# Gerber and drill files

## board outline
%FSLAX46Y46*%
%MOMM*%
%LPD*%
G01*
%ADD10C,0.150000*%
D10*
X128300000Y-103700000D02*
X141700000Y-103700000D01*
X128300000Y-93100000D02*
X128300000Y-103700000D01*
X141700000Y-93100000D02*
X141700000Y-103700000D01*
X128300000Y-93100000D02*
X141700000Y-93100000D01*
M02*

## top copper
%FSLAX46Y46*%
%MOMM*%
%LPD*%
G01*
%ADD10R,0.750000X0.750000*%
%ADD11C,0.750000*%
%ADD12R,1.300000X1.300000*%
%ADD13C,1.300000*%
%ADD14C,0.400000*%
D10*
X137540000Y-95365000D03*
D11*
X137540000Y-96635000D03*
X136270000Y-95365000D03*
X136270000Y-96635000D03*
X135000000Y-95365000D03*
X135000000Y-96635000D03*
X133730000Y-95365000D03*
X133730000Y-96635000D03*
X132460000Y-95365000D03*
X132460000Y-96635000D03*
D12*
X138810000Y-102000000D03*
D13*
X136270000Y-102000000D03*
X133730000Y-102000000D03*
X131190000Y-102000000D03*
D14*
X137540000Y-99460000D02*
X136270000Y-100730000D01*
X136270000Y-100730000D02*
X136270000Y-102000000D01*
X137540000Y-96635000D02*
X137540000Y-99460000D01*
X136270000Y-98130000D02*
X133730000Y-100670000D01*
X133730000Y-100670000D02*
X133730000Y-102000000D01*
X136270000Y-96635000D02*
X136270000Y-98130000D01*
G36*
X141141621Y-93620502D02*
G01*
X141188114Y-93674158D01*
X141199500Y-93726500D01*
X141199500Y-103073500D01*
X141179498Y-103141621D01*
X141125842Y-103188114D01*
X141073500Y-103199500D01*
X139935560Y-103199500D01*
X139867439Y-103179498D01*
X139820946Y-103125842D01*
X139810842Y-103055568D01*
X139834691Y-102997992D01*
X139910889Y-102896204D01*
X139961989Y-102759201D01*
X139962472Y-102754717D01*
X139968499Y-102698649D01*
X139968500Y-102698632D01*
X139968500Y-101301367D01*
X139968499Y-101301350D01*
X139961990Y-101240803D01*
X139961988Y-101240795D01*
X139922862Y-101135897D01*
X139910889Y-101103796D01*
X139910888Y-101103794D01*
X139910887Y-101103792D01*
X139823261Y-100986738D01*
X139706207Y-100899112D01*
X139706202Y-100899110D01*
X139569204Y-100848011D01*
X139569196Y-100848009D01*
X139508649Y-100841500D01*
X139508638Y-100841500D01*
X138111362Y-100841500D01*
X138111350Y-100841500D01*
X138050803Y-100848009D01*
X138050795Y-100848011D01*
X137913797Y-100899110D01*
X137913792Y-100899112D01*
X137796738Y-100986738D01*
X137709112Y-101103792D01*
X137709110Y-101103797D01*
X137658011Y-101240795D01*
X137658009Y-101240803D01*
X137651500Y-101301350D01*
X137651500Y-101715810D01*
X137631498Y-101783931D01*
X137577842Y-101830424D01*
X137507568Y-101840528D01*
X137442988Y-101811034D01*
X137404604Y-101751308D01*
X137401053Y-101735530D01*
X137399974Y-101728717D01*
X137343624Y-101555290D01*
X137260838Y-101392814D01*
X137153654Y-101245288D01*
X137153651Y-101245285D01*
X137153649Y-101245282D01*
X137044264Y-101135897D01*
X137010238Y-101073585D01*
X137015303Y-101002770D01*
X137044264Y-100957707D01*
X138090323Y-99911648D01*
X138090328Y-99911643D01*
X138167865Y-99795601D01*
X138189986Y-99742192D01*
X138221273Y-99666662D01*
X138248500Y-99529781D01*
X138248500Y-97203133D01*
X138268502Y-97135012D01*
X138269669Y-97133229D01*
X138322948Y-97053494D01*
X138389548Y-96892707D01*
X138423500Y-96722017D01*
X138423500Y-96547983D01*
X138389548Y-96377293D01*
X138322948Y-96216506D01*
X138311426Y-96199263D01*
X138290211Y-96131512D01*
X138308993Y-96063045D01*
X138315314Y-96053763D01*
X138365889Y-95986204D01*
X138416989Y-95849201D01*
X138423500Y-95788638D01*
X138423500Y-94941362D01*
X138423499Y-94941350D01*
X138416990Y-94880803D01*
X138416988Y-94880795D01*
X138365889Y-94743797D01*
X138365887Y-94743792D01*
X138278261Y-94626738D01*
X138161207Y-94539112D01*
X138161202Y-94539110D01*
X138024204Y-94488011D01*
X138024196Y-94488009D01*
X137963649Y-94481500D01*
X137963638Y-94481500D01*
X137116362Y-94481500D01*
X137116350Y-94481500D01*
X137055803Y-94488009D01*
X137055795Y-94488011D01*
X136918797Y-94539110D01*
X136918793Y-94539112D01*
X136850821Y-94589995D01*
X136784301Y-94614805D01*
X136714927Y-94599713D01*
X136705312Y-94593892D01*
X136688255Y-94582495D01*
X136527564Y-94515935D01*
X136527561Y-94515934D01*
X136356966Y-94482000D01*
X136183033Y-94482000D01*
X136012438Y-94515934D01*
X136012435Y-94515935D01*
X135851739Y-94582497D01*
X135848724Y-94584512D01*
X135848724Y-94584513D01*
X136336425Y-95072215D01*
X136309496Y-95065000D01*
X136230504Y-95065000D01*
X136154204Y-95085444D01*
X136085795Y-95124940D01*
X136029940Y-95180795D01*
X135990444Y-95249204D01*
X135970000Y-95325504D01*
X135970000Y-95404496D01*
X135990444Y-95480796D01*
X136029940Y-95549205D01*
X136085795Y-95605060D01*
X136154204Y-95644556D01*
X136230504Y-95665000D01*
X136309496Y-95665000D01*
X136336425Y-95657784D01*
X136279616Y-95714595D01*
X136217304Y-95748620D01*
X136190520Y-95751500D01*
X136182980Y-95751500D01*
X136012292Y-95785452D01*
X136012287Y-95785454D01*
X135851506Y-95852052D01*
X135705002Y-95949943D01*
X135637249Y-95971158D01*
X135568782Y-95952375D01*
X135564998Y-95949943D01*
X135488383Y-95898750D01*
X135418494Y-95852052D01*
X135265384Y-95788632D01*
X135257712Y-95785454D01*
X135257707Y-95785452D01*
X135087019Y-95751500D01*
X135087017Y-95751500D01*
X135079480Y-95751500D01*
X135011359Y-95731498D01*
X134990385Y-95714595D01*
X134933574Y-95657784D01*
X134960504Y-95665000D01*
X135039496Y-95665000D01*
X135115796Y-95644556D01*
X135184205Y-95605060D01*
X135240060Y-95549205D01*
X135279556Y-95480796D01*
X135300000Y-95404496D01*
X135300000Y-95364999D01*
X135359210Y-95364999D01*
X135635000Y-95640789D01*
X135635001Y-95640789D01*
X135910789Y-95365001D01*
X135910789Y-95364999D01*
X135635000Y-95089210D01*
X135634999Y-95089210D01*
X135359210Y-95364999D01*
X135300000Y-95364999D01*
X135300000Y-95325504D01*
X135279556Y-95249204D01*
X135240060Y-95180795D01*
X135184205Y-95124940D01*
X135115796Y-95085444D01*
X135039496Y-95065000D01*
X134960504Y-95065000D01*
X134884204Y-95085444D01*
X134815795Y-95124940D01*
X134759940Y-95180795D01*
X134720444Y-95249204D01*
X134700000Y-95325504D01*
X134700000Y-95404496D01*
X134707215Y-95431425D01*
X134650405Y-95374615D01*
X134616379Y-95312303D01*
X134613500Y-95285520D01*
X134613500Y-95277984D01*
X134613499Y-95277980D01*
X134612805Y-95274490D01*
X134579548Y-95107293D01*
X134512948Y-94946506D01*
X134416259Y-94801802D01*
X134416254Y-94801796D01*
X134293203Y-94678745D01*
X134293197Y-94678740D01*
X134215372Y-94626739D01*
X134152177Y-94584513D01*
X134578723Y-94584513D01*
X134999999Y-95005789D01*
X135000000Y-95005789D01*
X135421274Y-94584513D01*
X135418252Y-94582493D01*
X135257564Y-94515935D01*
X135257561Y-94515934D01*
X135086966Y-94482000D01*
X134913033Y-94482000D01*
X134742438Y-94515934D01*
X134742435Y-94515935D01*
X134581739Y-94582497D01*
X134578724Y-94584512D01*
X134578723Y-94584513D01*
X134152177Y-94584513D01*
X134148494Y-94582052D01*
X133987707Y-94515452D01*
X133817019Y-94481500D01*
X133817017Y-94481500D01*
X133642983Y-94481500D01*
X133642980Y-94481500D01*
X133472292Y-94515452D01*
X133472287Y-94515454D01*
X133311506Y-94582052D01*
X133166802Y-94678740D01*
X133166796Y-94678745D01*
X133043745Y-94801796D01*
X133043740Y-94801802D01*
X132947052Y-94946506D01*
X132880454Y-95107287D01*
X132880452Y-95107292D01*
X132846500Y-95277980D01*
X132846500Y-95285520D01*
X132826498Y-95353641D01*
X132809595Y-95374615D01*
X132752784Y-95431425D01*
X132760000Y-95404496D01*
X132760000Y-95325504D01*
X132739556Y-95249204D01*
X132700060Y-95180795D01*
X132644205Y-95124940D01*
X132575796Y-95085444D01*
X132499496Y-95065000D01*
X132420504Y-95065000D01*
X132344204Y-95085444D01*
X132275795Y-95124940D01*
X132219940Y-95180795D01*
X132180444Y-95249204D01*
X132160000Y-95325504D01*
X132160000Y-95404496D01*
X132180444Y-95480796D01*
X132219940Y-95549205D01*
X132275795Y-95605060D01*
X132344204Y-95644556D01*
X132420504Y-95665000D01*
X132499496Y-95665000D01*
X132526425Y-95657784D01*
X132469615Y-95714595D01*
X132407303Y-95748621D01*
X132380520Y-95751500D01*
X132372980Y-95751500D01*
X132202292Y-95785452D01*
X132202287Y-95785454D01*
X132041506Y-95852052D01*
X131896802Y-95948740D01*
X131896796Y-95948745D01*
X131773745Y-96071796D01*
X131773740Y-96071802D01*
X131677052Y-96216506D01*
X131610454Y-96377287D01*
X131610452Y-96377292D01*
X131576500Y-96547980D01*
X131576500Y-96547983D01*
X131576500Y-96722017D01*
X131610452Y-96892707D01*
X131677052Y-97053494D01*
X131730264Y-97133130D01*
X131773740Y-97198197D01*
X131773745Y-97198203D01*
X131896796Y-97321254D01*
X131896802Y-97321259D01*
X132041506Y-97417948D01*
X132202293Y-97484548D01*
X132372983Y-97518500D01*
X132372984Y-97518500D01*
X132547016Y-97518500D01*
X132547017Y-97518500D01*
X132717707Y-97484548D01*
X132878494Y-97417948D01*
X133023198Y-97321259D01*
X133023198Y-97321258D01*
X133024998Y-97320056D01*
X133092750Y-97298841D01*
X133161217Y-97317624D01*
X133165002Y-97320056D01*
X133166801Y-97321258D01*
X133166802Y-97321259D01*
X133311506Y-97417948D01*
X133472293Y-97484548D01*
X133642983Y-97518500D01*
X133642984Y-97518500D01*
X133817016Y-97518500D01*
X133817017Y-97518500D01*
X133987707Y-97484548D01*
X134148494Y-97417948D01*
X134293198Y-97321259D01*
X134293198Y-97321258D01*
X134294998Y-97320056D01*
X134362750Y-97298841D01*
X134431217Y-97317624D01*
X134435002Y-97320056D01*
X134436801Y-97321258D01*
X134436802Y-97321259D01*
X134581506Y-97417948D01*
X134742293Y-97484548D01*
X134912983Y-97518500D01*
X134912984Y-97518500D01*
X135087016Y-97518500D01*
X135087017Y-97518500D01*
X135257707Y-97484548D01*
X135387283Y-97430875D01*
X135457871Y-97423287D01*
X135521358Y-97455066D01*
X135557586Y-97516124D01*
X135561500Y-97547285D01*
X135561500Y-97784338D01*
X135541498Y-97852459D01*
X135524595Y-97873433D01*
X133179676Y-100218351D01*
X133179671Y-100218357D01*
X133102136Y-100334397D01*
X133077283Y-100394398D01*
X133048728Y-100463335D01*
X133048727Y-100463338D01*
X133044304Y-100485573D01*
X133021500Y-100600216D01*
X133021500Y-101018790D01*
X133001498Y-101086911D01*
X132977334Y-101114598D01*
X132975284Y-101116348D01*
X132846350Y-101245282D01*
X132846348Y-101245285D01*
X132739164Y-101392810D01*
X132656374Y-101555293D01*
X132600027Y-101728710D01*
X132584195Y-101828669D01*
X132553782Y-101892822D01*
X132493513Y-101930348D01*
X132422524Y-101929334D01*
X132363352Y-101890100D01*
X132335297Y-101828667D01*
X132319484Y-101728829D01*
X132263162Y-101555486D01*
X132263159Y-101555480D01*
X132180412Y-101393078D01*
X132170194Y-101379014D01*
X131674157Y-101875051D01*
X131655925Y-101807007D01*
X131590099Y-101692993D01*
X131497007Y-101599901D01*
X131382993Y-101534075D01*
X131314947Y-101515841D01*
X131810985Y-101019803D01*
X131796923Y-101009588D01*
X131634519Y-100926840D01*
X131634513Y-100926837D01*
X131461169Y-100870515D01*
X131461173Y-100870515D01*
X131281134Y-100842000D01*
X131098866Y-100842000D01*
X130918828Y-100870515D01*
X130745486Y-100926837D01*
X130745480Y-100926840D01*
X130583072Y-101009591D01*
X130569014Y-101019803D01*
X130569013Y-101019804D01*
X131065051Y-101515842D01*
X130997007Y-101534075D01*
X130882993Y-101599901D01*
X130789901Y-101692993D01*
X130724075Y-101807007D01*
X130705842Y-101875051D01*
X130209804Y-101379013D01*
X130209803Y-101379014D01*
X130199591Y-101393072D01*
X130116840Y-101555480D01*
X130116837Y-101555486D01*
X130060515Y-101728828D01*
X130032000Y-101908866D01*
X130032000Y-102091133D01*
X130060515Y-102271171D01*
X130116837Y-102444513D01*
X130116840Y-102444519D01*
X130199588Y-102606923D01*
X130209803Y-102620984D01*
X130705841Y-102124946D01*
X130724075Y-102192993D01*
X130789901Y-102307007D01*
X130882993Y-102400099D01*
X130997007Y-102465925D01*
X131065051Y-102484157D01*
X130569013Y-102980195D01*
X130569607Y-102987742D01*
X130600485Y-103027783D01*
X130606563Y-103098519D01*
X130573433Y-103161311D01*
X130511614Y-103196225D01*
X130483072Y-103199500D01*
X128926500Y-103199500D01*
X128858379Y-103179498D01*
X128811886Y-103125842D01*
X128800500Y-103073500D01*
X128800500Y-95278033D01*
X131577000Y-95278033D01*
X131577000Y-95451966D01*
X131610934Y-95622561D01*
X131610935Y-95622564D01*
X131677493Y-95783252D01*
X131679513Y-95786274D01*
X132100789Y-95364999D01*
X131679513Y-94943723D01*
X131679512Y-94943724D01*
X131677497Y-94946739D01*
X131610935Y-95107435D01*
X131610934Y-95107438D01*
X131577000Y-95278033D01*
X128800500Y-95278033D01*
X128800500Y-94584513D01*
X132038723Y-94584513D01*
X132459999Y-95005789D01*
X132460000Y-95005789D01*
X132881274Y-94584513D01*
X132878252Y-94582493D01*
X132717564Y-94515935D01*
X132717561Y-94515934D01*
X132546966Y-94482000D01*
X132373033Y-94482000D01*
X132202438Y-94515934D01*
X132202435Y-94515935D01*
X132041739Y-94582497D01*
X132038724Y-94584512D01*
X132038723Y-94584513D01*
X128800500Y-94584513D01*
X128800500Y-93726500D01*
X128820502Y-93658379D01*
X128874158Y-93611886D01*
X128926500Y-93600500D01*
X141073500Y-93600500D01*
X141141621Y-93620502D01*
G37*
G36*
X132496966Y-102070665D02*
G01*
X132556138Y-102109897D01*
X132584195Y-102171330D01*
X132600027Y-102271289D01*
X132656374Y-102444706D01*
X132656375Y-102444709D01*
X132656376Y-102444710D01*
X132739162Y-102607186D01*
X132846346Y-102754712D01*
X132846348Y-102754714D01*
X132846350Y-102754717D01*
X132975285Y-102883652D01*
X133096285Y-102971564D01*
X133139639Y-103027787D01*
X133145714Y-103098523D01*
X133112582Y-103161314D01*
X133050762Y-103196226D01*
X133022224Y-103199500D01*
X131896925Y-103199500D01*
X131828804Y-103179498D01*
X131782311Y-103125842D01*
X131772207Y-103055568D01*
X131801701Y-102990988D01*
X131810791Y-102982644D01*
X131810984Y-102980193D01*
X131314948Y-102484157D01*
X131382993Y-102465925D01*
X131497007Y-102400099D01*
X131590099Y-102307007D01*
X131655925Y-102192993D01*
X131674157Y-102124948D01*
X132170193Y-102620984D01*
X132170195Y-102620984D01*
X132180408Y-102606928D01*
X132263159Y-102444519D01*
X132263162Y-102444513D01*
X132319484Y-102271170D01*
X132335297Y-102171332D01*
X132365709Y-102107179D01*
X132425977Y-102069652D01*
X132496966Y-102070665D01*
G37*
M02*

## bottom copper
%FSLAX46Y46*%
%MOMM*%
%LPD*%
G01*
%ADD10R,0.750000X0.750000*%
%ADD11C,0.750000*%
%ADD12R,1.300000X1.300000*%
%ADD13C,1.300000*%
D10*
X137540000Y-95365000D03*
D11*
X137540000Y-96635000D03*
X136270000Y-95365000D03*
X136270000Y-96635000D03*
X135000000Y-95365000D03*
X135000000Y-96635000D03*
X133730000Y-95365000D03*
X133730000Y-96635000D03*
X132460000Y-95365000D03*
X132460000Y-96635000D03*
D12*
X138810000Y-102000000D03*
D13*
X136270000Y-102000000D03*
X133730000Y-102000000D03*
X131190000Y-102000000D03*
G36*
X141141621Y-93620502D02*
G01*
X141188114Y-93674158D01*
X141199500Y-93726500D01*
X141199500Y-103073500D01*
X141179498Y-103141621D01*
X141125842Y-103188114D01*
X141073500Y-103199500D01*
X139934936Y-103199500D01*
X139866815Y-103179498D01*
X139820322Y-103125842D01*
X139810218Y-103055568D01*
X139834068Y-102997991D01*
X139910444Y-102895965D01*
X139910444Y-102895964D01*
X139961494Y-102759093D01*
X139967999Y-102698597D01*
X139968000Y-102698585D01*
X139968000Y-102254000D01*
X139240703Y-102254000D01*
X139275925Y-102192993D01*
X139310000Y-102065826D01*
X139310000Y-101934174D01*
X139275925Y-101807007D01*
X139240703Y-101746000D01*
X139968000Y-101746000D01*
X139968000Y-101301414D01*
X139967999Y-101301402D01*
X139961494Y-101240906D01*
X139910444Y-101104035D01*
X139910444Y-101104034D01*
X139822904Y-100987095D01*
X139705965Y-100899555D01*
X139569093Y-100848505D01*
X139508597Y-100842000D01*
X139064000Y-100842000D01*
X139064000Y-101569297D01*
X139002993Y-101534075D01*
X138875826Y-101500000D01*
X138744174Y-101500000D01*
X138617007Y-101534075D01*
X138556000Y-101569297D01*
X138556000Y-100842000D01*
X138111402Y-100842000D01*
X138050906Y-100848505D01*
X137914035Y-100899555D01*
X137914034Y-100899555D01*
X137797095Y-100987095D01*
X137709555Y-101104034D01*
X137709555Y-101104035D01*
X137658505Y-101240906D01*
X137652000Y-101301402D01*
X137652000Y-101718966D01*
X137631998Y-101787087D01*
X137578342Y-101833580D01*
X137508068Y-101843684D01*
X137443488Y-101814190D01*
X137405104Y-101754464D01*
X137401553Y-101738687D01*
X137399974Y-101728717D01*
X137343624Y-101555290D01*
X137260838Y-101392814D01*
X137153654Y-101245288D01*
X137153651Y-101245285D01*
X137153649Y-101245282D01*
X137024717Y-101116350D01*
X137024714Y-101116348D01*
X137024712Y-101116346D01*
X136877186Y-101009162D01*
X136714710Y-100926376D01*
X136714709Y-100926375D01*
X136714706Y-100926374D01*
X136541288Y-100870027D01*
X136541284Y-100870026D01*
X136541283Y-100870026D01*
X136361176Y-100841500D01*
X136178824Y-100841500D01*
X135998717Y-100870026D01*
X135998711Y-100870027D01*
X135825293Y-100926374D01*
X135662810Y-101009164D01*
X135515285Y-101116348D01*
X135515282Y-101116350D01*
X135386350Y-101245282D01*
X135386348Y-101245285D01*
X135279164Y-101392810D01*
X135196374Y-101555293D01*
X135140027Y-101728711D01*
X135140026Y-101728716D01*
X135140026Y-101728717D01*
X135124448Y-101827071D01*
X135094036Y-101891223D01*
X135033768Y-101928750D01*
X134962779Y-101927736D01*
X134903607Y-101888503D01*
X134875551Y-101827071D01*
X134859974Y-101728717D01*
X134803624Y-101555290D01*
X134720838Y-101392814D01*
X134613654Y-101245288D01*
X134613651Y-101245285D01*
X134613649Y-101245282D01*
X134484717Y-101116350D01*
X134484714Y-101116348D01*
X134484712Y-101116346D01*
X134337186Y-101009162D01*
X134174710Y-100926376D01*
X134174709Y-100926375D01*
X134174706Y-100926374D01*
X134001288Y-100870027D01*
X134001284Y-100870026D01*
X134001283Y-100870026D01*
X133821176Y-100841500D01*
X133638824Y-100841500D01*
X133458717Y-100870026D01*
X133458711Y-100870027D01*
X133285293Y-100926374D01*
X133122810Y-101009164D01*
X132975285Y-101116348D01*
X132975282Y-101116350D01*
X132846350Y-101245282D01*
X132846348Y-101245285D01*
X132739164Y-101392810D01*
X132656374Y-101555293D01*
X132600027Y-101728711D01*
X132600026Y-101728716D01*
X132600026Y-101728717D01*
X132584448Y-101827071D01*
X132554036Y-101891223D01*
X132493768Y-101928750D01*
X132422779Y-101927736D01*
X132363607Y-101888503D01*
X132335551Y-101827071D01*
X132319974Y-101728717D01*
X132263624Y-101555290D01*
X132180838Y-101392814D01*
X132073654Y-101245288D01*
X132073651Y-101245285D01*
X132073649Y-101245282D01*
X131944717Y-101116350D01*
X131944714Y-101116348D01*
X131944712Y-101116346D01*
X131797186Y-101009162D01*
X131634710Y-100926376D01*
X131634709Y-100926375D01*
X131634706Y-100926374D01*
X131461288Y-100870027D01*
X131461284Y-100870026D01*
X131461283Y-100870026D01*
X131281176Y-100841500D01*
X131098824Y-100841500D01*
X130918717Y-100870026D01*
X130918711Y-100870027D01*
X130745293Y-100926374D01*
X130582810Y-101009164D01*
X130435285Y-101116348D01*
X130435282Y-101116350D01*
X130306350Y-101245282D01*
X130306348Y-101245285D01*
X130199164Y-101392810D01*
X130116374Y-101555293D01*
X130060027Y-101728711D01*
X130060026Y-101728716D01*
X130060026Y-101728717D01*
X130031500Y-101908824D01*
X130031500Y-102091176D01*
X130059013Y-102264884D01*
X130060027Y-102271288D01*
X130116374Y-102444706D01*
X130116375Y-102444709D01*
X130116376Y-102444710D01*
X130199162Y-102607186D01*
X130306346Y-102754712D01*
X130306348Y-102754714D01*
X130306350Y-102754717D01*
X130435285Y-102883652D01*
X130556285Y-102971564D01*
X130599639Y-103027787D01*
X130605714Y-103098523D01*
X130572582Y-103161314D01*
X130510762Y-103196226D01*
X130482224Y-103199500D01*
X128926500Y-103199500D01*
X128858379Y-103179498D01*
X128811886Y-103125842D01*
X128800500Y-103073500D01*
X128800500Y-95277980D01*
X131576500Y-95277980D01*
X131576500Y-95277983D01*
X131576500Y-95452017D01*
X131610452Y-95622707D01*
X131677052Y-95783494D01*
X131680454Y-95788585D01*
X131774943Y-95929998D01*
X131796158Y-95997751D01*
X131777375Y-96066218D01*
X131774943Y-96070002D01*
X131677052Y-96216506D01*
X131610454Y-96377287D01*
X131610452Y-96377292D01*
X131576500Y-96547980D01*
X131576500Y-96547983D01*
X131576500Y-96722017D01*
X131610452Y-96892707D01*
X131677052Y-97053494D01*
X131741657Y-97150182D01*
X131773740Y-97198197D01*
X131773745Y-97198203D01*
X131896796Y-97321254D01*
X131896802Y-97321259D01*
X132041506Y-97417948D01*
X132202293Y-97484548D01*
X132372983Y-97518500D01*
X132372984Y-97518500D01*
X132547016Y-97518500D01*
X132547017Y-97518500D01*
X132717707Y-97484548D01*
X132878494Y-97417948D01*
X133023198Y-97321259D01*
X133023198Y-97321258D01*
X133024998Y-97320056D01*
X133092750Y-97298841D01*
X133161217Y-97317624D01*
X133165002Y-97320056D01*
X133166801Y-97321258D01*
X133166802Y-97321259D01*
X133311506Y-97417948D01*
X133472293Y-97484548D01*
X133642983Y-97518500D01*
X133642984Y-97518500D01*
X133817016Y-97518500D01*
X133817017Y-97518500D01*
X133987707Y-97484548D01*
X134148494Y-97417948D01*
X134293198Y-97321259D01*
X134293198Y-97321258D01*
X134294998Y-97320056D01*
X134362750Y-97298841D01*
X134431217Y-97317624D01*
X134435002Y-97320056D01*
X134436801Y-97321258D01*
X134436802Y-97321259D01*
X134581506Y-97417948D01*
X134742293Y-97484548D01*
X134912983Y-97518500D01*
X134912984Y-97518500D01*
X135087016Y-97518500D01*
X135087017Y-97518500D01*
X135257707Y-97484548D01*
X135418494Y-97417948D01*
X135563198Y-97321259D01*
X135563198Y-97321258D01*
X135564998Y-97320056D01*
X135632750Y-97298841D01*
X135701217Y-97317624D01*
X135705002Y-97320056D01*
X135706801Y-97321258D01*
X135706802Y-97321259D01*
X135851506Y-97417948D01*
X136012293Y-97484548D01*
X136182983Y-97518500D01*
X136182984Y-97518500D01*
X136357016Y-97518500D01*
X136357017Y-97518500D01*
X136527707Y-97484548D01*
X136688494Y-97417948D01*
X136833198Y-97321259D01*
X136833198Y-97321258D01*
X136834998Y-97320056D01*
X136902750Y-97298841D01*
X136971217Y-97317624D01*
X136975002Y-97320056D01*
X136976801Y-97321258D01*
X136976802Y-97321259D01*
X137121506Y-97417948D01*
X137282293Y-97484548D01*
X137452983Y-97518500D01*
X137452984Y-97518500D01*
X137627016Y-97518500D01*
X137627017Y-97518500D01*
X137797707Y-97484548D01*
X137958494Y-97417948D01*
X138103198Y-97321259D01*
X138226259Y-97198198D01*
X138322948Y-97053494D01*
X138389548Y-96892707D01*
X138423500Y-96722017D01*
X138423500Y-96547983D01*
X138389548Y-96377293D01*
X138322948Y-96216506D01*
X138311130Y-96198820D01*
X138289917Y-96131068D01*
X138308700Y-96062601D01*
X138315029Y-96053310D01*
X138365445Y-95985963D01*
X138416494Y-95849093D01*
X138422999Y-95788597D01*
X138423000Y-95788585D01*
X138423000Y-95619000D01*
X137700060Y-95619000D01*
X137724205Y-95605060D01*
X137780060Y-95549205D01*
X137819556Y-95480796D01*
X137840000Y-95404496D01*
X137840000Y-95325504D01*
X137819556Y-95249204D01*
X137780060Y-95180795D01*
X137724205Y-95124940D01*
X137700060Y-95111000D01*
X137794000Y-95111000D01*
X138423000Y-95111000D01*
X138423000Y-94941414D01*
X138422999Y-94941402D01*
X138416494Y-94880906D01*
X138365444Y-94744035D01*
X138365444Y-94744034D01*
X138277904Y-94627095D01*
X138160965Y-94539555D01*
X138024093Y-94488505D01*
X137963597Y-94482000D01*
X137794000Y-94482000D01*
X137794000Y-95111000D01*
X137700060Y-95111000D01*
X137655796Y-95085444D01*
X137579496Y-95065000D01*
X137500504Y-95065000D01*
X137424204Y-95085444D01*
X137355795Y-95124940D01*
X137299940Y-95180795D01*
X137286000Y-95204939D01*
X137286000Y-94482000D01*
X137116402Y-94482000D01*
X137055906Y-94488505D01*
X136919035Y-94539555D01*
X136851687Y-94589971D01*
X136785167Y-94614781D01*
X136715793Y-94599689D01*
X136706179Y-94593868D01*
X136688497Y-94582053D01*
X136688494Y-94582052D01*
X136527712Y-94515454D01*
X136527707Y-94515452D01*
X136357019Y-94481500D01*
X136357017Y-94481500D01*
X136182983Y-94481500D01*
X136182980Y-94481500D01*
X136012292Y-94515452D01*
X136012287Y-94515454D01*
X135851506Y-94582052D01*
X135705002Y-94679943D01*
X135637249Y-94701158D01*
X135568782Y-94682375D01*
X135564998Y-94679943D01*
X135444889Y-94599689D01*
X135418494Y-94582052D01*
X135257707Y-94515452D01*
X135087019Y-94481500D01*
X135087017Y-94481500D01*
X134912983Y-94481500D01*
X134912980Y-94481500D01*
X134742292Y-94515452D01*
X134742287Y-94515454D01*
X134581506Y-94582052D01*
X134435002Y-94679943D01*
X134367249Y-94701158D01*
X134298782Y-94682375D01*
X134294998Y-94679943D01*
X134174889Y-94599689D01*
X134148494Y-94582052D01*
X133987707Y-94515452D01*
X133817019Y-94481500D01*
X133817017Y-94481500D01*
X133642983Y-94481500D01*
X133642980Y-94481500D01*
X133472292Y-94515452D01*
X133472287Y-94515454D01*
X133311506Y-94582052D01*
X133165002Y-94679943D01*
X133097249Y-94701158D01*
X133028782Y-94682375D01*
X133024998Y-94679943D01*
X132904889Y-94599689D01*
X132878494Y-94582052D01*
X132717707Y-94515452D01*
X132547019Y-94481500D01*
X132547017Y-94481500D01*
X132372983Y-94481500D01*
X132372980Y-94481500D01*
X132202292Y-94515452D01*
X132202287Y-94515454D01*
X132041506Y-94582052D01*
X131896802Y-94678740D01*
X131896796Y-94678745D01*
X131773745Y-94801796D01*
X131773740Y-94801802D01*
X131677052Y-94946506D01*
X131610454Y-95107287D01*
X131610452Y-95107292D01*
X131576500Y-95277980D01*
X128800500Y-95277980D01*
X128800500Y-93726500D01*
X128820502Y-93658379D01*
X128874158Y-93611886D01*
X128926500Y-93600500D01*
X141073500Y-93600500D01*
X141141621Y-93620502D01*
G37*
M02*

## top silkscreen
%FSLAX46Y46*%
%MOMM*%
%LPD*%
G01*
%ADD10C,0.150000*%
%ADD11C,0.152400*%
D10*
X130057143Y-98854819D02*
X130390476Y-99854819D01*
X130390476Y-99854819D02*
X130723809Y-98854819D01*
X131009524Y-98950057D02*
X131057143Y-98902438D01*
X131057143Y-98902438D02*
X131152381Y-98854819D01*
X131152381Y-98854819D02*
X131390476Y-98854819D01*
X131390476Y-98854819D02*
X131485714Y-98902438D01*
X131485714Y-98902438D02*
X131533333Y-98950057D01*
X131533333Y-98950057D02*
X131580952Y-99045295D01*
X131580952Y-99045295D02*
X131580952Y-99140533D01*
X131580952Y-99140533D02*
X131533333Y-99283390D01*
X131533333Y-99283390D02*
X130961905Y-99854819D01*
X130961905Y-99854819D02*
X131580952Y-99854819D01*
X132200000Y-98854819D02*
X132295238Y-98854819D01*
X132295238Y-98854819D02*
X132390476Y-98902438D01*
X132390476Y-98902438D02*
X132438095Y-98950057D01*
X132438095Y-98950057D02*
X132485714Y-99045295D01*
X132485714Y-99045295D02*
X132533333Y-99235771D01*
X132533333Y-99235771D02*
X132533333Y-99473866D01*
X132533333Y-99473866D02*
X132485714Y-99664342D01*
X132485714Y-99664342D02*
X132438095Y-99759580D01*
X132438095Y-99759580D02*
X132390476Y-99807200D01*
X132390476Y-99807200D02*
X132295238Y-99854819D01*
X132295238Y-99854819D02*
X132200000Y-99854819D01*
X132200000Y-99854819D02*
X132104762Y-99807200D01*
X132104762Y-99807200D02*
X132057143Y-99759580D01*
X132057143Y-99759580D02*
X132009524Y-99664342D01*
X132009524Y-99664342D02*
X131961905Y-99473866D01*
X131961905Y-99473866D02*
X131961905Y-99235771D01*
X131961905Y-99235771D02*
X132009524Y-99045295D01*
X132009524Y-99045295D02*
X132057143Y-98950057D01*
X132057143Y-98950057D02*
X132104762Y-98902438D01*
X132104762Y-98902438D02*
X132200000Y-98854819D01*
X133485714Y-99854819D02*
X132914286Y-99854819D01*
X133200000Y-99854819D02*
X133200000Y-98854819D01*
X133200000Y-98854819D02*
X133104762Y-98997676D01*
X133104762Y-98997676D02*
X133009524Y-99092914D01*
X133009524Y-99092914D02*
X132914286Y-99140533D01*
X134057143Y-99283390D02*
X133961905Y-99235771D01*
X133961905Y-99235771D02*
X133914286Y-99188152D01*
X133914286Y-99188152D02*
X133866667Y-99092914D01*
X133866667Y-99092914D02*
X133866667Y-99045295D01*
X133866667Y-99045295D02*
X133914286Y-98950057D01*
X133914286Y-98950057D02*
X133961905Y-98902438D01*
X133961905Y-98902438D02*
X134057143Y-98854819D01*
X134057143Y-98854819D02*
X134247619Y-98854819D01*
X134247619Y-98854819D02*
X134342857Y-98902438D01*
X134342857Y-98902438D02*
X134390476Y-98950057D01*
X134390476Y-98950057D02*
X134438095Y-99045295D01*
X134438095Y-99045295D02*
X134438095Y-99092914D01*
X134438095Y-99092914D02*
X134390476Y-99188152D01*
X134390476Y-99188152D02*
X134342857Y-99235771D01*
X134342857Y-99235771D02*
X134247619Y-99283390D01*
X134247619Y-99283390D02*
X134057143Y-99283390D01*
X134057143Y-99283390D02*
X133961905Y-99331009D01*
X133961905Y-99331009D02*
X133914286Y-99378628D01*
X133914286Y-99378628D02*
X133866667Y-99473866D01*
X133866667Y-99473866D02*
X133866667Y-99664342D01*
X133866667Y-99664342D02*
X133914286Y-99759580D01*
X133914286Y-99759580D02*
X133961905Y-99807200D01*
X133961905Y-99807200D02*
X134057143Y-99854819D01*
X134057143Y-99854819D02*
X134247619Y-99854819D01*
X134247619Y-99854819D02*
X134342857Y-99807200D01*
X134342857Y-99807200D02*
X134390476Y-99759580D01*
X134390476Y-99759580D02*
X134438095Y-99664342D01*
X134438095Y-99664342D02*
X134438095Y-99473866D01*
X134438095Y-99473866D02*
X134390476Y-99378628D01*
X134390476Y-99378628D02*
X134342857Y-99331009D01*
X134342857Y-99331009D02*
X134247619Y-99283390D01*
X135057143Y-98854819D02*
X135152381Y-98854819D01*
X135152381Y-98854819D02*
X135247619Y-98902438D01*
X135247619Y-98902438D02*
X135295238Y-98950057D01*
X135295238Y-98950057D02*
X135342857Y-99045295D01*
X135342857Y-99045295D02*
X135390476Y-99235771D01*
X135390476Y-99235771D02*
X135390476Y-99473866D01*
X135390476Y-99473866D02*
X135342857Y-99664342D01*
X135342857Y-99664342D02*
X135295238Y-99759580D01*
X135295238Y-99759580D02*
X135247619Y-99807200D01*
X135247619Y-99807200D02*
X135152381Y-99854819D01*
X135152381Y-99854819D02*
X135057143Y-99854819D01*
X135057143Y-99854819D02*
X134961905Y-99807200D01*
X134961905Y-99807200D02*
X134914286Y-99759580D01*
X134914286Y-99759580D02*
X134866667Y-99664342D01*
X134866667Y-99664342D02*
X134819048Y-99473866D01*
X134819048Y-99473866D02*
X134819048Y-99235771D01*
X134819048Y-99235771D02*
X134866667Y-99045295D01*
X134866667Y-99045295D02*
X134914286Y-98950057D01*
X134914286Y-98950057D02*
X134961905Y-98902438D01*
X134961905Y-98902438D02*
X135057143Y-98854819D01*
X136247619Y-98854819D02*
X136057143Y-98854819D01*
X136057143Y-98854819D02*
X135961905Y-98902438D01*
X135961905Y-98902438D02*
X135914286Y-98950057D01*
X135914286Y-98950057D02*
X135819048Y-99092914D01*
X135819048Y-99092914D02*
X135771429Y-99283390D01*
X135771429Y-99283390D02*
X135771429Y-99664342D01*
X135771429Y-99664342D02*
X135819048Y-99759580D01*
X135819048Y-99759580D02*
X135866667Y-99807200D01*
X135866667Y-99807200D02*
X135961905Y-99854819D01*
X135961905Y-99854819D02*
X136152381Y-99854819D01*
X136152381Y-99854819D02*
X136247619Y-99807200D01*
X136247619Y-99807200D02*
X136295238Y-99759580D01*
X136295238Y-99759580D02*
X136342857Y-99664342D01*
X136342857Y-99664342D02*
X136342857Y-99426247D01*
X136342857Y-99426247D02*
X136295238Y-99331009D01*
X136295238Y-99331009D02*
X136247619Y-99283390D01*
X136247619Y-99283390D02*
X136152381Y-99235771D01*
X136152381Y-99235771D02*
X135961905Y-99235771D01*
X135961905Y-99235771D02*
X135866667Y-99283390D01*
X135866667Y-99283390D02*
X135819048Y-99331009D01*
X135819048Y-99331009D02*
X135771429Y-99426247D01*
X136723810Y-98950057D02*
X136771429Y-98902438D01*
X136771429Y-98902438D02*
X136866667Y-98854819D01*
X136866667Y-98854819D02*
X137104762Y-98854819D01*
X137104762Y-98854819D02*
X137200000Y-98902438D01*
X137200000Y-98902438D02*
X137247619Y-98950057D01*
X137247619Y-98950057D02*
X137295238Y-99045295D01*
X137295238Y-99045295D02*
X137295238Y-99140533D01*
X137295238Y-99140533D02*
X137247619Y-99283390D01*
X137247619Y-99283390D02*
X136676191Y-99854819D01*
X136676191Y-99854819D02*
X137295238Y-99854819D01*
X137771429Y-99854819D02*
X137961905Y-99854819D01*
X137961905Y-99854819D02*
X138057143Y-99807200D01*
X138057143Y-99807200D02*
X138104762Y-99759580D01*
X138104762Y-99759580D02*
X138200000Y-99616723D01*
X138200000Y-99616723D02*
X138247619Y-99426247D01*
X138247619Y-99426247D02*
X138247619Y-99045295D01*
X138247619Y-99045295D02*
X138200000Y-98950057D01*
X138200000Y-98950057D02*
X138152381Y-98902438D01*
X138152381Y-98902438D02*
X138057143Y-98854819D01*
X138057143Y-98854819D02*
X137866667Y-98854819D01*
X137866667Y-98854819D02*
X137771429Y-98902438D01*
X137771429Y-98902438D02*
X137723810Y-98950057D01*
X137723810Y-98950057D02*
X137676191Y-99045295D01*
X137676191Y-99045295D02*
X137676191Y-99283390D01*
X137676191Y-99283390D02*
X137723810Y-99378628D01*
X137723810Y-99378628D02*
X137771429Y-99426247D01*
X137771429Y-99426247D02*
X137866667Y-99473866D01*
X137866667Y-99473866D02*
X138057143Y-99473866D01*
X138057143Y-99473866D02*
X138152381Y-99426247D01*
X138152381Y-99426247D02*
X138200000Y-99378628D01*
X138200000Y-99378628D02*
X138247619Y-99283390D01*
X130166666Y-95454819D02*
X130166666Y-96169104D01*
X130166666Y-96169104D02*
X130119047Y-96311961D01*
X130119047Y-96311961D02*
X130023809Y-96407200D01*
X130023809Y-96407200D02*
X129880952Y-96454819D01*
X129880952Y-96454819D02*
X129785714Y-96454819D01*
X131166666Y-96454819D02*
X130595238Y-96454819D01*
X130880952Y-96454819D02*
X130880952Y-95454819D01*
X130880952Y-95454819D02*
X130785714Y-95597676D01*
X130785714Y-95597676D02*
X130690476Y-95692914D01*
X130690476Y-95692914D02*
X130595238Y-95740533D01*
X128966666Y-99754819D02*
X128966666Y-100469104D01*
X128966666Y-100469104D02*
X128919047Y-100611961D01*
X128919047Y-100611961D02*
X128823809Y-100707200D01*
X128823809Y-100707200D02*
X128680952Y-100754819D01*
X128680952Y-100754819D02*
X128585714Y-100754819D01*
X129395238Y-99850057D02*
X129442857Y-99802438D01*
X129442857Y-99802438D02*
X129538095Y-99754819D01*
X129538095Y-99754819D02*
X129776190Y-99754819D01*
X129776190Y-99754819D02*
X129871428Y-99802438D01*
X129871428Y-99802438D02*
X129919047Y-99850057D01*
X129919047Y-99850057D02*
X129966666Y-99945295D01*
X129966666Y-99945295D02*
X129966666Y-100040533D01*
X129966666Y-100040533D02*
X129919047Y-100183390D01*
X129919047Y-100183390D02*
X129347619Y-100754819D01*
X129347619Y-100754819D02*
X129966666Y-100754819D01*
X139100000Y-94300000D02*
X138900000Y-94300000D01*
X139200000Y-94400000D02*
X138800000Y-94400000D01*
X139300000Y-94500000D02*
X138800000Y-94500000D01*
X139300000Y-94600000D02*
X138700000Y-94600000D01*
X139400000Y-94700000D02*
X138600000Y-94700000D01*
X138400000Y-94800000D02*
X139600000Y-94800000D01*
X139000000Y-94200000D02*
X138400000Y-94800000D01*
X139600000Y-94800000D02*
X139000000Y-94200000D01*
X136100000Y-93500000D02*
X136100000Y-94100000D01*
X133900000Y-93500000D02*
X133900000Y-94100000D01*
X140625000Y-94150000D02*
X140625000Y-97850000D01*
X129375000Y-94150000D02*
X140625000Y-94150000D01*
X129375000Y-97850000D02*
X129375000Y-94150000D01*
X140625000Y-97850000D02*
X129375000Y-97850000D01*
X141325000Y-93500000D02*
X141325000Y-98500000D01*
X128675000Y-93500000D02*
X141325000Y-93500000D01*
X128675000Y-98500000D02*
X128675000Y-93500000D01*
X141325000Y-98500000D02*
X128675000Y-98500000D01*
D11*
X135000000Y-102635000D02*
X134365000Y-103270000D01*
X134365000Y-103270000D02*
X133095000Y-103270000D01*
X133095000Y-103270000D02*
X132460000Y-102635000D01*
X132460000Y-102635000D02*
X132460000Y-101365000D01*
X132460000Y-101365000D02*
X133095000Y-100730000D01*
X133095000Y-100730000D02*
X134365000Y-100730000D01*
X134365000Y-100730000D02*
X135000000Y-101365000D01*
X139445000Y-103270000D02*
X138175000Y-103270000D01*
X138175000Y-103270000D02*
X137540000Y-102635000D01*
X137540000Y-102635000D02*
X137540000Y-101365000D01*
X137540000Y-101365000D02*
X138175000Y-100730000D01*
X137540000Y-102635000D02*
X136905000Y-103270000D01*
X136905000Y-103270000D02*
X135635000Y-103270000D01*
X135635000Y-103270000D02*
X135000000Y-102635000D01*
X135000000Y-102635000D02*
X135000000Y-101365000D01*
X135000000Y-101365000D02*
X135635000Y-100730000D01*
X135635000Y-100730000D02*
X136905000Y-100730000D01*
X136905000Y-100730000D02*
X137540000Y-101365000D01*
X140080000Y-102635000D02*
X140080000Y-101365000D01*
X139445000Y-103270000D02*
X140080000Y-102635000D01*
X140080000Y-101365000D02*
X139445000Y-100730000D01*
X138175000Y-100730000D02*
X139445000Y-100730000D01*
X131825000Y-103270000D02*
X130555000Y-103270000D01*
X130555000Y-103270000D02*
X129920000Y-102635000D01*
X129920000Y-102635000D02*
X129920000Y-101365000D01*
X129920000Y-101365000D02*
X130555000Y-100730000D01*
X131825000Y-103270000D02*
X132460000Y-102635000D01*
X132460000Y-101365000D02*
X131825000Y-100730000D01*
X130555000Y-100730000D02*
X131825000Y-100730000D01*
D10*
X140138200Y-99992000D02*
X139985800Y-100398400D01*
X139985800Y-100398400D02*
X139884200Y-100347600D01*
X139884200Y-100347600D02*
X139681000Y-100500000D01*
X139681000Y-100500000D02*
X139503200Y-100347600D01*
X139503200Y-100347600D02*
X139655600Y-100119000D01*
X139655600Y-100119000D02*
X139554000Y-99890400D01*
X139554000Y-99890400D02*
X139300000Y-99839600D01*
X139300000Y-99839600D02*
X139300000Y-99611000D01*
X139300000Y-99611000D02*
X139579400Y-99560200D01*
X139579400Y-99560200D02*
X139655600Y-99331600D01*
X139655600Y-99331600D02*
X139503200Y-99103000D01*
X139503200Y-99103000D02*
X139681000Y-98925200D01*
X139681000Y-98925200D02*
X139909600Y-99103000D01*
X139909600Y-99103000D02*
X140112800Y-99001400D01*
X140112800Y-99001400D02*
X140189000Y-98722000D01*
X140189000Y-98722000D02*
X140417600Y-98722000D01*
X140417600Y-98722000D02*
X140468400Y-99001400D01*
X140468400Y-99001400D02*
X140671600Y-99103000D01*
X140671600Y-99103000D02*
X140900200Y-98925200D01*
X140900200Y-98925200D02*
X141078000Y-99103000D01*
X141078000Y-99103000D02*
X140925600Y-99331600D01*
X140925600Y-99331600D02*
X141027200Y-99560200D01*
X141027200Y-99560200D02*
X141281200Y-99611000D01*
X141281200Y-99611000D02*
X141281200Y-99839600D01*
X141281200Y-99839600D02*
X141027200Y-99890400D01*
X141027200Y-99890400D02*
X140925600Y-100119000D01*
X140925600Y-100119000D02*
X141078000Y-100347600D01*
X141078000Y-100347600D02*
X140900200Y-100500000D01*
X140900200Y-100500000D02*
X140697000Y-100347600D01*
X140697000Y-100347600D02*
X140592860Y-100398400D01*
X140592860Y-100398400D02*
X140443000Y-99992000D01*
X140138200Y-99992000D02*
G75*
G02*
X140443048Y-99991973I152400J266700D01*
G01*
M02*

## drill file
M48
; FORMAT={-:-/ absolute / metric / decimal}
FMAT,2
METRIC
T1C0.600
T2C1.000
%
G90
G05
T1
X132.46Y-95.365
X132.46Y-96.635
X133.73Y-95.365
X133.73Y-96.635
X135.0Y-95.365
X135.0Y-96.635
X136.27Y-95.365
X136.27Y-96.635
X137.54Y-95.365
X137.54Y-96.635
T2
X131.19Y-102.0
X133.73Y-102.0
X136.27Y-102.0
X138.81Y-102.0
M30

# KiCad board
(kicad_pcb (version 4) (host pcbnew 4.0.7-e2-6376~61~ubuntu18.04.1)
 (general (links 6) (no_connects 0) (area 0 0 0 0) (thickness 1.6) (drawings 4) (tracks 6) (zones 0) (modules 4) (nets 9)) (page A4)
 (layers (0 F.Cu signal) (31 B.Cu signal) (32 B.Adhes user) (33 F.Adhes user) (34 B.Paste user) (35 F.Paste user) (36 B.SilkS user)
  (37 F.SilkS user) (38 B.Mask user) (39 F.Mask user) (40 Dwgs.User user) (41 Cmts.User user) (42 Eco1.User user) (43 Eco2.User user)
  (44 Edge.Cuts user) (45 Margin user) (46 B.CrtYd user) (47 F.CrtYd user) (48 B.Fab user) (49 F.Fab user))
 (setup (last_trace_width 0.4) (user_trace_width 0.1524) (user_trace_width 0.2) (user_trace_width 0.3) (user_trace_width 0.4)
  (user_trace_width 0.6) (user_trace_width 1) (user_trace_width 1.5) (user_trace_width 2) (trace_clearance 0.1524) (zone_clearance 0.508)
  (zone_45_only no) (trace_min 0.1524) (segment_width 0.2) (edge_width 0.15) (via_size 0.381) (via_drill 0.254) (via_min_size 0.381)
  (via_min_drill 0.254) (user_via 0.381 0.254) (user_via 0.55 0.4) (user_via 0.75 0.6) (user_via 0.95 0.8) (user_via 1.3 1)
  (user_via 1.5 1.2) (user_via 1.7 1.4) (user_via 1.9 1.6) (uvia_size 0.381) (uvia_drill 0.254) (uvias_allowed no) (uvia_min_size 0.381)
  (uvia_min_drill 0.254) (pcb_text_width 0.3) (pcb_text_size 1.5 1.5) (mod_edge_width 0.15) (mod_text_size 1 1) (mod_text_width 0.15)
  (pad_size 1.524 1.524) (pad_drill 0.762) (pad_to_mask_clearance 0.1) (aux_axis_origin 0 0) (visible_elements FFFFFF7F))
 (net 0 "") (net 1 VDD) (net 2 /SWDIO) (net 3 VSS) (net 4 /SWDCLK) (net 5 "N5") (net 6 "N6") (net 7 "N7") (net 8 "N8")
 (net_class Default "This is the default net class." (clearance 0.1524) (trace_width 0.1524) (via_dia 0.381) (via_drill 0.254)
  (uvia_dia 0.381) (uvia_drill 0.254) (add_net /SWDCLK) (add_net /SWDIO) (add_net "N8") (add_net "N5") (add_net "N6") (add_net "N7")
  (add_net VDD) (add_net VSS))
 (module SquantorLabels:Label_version (layer F.Cu) (at 135 99.4)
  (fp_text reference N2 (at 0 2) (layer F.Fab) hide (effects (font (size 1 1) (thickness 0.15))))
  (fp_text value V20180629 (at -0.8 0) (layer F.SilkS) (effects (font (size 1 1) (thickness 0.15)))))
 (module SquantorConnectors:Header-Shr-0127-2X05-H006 (layer F.Cu) (at 135 96 180)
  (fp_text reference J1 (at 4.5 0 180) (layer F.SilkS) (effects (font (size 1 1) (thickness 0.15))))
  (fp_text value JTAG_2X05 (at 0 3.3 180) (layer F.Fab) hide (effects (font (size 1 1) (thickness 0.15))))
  (fp_line (start -4.1 1.7) (end -3.9 1.7) (layer F.SilkS) (width 0.15))
  (fp_line (start -4.2 1.6) (end -3.8 1.6) (layer F.SilkS) (width 0.15))
  (fp_line (start -4.3 1.5) (end -3.8 1.5) (layer F.SilkS) (width 0.15))
  (fp_line (start -4.3 1.4) (end -3.7 1.4) (layer F.SilkS) (width 0.15))
  (fp_line (start -4.4 1.3) (end -3.6 1.3) (layer F.SilkS) (width 0.15))
  (fp_line (start -3.4 1.2) (end -4.6 1.2) (layer F.SilkS) (width 0.15))
  (fp_line (start -4 1.8) (end -3.4 1.2) (layer F.SilkS) (width 0.15))
  (fp_line (start -4.6 1.2) (end -4 1.8) (layer F.SilkS) (width 0.15))
  (fp_line (start -1.1 2.5) (end -1.1 1.9) (layer F.SilkS) (width 0.15))
  (fp_line (start 1.1 2.5) (end 1.1 1.9) (layer F.SilkS) (width 0.15))
  (fp_line (start -5.625 1.85) (end -5.625 -1.85) (layer F.SilkS) (width 0.15))
  (fp_line (start 5.625 1.85) (end -5.625 1.85) (layer F.SilkS) (width 0.15))
  (fp_line (start 5.625 -1.85) (end 5.625 1.85) (layer F.SilkS) (width 0.15))
  (fp_line (start -5.625 -1.85) (end 5.625 -1.85) (layer F.SilkS) (width 0.15))
  (fp_line (start -6.325 2.5) (end -6.325 -2.5) (layer F.SilkS) (width 0.15))
  (fp_line (start 6.325 2.5) (end -6.325 2.5) (layer F.SilkS) (width 0.15))
  (fp_line (start 6.325 -2.5) (end 6.325 2.5) (layer F.SilkS) (width 0.15))
  (fp_line (start -6.325 -2.5) (end 6.325 -2.5) (layer F.SilkS) (width 0.15))
  (pad 1 thru_hole rect (at -2.54 0.635 180) (size 0.75 0.75) (drill 0.6) (layers *.Cu *.Mask) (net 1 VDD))
  (pad 2 thru_hole circle (at -2.54 -0.635 180) (size 0.75 0.75) (drill 0.6) (layers *.Cu *.Mask) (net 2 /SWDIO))
  (pad 3 thru_hole circle (at -1.27 0.635 180) (size 0.75 0.75) (drill 0.6) (layers *.Cu *.Mask) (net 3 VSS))
  (pad 4 thru_hole circle (at -1.27 -0.635 180) (size 0.75 0.75) (drill 0.6) (layers *.Cu *.Mask) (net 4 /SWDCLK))
  (pad 5 thru_hole circle (at 0 0.635 180) (size 0.75 0.75) (drill 0.6) (layers *.Cu *.Mask) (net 3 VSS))
  (pad 6 thru_hole circle (at 0 -0.635 180) (size 0.75 0.75) (drill 0.6) (layers *.Cu *.Mask) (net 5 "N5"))
  (pad 7 thru_hole circle (at 1.27 0.635 180) (size 0.75 0.75) (drill 0.6) (layers *.Cu *.Mask) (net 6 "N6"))
  (pad 8 thru_hole circle (at 1.27 -0.635 180) (size 0.75 0.75) (drill 0.6) (layers *.Cu *.Mask) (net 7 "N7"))
  (pad 9 thru_hole circle (at 2.54 0.635 180) (size 0.75 0.75) (drill 0.6) (layers *.Cu *.Mask) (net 3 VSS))
  (pad 10 thru_hole circle (at 2.54 -0.635 180) (size 0.75 0.75) (drill 0.6) (layers *.Cu *.Mask) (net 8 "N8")))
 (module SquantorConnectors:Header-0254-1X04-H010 (layer F.Cu) (at 135 102 180)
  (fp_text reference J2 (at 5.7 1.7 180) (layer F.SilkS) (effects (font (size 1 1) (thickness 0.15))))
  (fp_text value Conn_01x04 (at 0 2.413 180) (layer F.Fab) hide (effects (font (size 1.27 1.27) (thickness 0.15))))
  (fp_line (start 0 -0.635) (end 0.635 -1.27) (layer F.SilkS) (width 0.1524))
  (fp_line (start 0.635 -1.27) (end 1.905 -1.27) (layer F.SilkS) (width 0.1524))
  (fp_line (start 1.905 -1.27) (end 2.54 -0.635) (layer F.SilkS) (width 0.1524))
  (fp_line (start 2.54 -0.635) (end 2.54 0.635) (layer F.SilkS) (width 0.1524))
  (fp_line (start 2.54 0.635) (end 1.905 1.27) (layer F.SilkS) (width 0.1524))
  (fp_line (start 1.905 1.27) (end 0.635 1.27) (layer F.SilkS) (width 0.1524))
  (fp_line (start 0.635 1.27) (end 0 0.635) (layer F.SilkS) (width 0.1524))
  (fp_line (start -4.445 -1.27) (end -3.175 -1.27) (layer F.SilkS) (width 0.1524))
  (fp_line (start -3.175 -1.27) (end -2.54 -0.635) (layer F.SilkS) (width 0.1524))
  (fp_line (start -2.54 -0.635) (end -2.54 0.635) (layer F.SilkS) (width 0.1524))
  (fp_line (start -2.54 0.635) (end -3.175 1.27) (layer F.SilkS) (width 0.1524))
  (fp_line (start -2.54 -0.635) (end -1.905 -1.27) (layer F.SilkS) (width 0.1524))
  (fp_line (start -1.905 -1.27) (end -0.635 -1.27) (layer F.SilkS) (width 0.1524))
  (fp_line (start -0.635 -1.27) (end 0 -0.635) (layer F.SilkS) (width 0.1524))
  (fp_line (start 0 -0.635) (end 0 0.635) (layer F.SilkS) (width 0.1524))
  (fp_line (start 0 0.635) (end -0.635 1.27) (layer F.SilkS) (width 0.1524))
  (fp_line (start -0.635 1.27) (end -1.905 1.27) (layer F.SilkS) (width 0.1524))
  (fp_line (start -1.905 1.27) (end -2.54 0.635) (layer F.SilkS) (width 0.1524))
  (fp_line (start -5.08 -0.635) (end -5.08 0.635) (layer F.SilkS) (width 0.1524))
  (fp_line (start -4.445 -1.27) (end -5.08 -0.635) (layer F.SilkS) (width 0.1524))
  (fp_line (start -5.08 0.635) (end -4.445 1.27) (layer F.SilkS) (width 0.1524))
  (fp_line (start -3.175 1.27) (end -4.445 1.27) (layer F.SilkS) (width 0.1524))
  (fp_line (start 3.175 -1.27) (end 4.445 -1.27) (layer F.SilkS) (width 0.1524))
  (fp_line (start 4.445 -1.27) (end 5.08 -0.635) (layer F.SilkS) (width 0.1524))
  (fp_line (start 5.08 -0.635) (end 5.08 0.635) (layer F.SilkS) (width 0.1524))
  (fp_line (start 5.08 0.635) (end 4.445 1.27) (layer F.SilkS) (width 0.1524))
  (fp_line (start 3.175 -1.27) (end 2.54 -0.635) (layer F.SilkS) (width 0.1524))
  (fp_line (start 2.54 0.635) (end 3.175 1.27) (layer F.SilkS) (width 0.1524))
  (fp_line (start 4.445 1.27) (end 3.175 1.27) (layer F.SilkS) (width 0.1524))
  (pad 1 thru_hole rect (at -3.81 0) (size 1.3 1.3) (drill 1) (layers *.Cu *.Mask) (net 1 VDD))
  (pad 2 thru_hole circle (at -1.27 0) (size 1.3 1.3) (drill 1) (layers *.Cu *.Mask) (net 2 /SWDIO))
  (pad 3 thru_hole circle (at 1.27 0) (size 1.3 1.3) (drill 1) (layers *.Cu *.Mask) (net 4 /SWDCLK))
  (pad 4 thru_hole circle (at 3.81 0) (size 1.3 1.3) (drill 1) (layers *.Cu *.Mask) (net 3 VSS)))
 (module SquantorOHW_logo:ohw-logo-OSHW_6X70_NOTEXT (layer F.Cu) (at 140.3 99.7)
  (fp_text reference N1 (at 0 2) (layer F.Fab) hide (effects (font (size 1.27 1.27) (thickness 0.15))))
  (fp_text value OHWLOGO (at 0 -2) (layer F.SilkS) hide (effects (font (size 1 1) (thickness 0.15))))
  (fp_line (start -0.1618 0.292) (end -0.3142 0.6984) (layer F.SilkS) (width 0.15))
  (fp_line (start -0.3142 0.6984) (end -0.4158 0.6476) (layer F.SilkS) (width 0.15))
  (fp_line (start -0.4158 0.6476) (end -0.619 0.8) (layer F.SilkS) (width 0.15))
  (fp_line (start -0.619 0.8) (end -0.7968 0.6476) (layer F.SilkS) (width 0.15))
  (fp_line (start -0.7968 0.6476) (end -0.6444 0.419) (layer F.SilkS) (width 0.15))
  (fp_line (start -0.6444 0.419) (end -0.746 0.1904) (layer F.SilkS) (width 0.15))
  (fp_line (start -0.746 0.1904) (end -1 0.1396) (layer F.SilkS) (width 0.15))
  (fp_line (start -1 0.1396) (end -1 -0.089) (layer F.SilkS) (width 0.15))
  (fp_line (start -1 -0.089) (end -0.7206 -0.1398) (layer F.SilkS) (width 0.15))
  (fp_line (start -0.7206 -0.1398) (end -0.6444 -0.3684) (layer F.SilkS) (width 0.15))
  (fp_line (start -0.6444 -0.3684) (end -0.7968 -0.597) (layer F.SilkS) (width 0.15))
  (fp_line (start -0.7968 -0.597) (end -0.619 -0.7748) (layer F.SilkS) (width 0.15))
  (fp_line (start -0.619 -0.7748) (end -0.3904 -0.597) (layer F.SilkS) (width 0.15))
  (fp_line (start -0.3904 -0.597) (end -0.1872 -0.6986) (layer F.SilkS) (width 0.15))
  (fp_line (start -0.1872 -0.6986) (end -0.111 -0.978) (layer F.SilkS) (width 0.15))
  (fp_line (start -0.111 -0.978) (end 0.1176 -0.978) (layer F.SilkS) (width 0.15))
  (fp_line (start 0.1176 -0.978) (end 0.1684 -0.6986) (layer F.SilkS) (width 0.15))
  (fp_line (start 0.1684 -0.6986) (end 0.3716 -0.597) (layer F.SilkS) (width 0.15))
  (fp_line (start 0.3716 -0.597) (end 0.6002 -0.7748) (layer F.SilkS) (width 0.15))
  (fp_line (start 0.6002 -0.7748) (end 0.778 -0.597) (layer F.SilkS) (width 0.15))
  (fp_line (start 0.778 -0.597) (end 0.6256 -0.3684) (layer F.SilkS) (width 0.15))
  (fp_line (start 0.6256 -0.3684) (end 0.7272 -0.1398) (layer F.SilkS) (width 0.15))
  (fp_line (start 0.7272 -0.1398) (end 0.9812 -0.089) (layer F.SilkS) (width 0.15))
  (fp_line (start 0.9812 -0.089) (end 0.9812 0.1396) (layer F.SilkS) (width 0.15))
  (fp_line (start 0.9812 0.1396) (end 0.7272 0.1904) (layer F.SilkS) (width 0.15))
  (fp_line (start 0.7272 0.1904) (end 0.6256 0.419) (layer F.SilkS) (width 0.15))
  (fp_line (start 0.6256 0.419) (end 0.778 0.6476) (layer F.SilkS) (width 0.15))
  (fp_line (start 0.778 0.6476) (end 0.6002 0.8) (layer F.SilkS) (width 0.15))
  (fp_line (start 0.6002 0.8) (end 0.397 0.6476) (layer F.SilkS) (width 0.15))
  (fp_line (start 0.397 0.6476) (end 0.29286 0.6984) (layer F.SilkS) (width 0.15))
  (fp_line (start 0.29286 0.6984) (end 0.143 0.292) (layer F.SilkS) (width 0.15))
  (fp_arc (start -0.0094 0.0253) (end -0.1618 0.292) (angle 300.5) (layer F.SilkS) (width 0.15)))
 (gr_line (start 128.3 103.7) (end 141.7 103.7) (layer Edge.Cuts) (width 0.15))
 (gr_line (start 128.3 93.1) (end 128.3 103.7) (layer Edge.Cuts) (width 0.15))
 (gr_line (start 141.7 93.1) (end 141.7 103.7) (layer Edge.Cuts) (width 0.15))
 (gr_line (start 128.3 93.1) (end 141.7 93.1) (layer Edge.Cuts) (width 0.15))
 (segment (start 137.54 99.46) (end 136.27 100.73) (width 0.4) (layer F.Cu) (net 2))
 (segment (start 136.27 100.73) (end 136.27 102) (width 0.4) (layer F.Cu) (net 2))
 (segment (start 137.54 96.635) (end 137.54 99.46) (width 0.4) (layer F.Cu) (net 2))
 (segment (start 136.27 98.13) (end 133.73 100.67) (width 0.4) (layer F.Cu) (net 4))
 (segment (start 133.73 100.67) (end 133.73 102) (width 0.4) (layer F.Cu) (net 4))
 (segment (start 136.27 96.635) (end 136.27 98.13) (width 0.4) (layer F.Cu) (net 4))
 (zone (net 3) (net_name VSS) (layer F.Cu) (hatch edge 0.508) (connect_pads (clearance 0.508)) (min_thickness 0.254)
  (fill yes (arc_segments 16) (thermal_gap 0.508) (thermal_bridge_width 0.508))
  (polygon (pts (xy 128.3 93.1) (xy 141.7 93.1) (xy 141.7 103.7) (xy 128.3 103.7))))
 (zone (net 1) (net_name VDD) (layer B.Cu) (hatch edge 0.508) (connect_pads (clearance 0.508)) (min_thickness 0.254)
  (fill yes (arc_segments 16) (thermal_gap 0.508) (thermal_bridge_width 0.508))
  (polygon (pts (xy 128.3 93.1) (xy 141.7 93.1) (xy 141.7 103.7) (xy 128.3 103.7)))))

